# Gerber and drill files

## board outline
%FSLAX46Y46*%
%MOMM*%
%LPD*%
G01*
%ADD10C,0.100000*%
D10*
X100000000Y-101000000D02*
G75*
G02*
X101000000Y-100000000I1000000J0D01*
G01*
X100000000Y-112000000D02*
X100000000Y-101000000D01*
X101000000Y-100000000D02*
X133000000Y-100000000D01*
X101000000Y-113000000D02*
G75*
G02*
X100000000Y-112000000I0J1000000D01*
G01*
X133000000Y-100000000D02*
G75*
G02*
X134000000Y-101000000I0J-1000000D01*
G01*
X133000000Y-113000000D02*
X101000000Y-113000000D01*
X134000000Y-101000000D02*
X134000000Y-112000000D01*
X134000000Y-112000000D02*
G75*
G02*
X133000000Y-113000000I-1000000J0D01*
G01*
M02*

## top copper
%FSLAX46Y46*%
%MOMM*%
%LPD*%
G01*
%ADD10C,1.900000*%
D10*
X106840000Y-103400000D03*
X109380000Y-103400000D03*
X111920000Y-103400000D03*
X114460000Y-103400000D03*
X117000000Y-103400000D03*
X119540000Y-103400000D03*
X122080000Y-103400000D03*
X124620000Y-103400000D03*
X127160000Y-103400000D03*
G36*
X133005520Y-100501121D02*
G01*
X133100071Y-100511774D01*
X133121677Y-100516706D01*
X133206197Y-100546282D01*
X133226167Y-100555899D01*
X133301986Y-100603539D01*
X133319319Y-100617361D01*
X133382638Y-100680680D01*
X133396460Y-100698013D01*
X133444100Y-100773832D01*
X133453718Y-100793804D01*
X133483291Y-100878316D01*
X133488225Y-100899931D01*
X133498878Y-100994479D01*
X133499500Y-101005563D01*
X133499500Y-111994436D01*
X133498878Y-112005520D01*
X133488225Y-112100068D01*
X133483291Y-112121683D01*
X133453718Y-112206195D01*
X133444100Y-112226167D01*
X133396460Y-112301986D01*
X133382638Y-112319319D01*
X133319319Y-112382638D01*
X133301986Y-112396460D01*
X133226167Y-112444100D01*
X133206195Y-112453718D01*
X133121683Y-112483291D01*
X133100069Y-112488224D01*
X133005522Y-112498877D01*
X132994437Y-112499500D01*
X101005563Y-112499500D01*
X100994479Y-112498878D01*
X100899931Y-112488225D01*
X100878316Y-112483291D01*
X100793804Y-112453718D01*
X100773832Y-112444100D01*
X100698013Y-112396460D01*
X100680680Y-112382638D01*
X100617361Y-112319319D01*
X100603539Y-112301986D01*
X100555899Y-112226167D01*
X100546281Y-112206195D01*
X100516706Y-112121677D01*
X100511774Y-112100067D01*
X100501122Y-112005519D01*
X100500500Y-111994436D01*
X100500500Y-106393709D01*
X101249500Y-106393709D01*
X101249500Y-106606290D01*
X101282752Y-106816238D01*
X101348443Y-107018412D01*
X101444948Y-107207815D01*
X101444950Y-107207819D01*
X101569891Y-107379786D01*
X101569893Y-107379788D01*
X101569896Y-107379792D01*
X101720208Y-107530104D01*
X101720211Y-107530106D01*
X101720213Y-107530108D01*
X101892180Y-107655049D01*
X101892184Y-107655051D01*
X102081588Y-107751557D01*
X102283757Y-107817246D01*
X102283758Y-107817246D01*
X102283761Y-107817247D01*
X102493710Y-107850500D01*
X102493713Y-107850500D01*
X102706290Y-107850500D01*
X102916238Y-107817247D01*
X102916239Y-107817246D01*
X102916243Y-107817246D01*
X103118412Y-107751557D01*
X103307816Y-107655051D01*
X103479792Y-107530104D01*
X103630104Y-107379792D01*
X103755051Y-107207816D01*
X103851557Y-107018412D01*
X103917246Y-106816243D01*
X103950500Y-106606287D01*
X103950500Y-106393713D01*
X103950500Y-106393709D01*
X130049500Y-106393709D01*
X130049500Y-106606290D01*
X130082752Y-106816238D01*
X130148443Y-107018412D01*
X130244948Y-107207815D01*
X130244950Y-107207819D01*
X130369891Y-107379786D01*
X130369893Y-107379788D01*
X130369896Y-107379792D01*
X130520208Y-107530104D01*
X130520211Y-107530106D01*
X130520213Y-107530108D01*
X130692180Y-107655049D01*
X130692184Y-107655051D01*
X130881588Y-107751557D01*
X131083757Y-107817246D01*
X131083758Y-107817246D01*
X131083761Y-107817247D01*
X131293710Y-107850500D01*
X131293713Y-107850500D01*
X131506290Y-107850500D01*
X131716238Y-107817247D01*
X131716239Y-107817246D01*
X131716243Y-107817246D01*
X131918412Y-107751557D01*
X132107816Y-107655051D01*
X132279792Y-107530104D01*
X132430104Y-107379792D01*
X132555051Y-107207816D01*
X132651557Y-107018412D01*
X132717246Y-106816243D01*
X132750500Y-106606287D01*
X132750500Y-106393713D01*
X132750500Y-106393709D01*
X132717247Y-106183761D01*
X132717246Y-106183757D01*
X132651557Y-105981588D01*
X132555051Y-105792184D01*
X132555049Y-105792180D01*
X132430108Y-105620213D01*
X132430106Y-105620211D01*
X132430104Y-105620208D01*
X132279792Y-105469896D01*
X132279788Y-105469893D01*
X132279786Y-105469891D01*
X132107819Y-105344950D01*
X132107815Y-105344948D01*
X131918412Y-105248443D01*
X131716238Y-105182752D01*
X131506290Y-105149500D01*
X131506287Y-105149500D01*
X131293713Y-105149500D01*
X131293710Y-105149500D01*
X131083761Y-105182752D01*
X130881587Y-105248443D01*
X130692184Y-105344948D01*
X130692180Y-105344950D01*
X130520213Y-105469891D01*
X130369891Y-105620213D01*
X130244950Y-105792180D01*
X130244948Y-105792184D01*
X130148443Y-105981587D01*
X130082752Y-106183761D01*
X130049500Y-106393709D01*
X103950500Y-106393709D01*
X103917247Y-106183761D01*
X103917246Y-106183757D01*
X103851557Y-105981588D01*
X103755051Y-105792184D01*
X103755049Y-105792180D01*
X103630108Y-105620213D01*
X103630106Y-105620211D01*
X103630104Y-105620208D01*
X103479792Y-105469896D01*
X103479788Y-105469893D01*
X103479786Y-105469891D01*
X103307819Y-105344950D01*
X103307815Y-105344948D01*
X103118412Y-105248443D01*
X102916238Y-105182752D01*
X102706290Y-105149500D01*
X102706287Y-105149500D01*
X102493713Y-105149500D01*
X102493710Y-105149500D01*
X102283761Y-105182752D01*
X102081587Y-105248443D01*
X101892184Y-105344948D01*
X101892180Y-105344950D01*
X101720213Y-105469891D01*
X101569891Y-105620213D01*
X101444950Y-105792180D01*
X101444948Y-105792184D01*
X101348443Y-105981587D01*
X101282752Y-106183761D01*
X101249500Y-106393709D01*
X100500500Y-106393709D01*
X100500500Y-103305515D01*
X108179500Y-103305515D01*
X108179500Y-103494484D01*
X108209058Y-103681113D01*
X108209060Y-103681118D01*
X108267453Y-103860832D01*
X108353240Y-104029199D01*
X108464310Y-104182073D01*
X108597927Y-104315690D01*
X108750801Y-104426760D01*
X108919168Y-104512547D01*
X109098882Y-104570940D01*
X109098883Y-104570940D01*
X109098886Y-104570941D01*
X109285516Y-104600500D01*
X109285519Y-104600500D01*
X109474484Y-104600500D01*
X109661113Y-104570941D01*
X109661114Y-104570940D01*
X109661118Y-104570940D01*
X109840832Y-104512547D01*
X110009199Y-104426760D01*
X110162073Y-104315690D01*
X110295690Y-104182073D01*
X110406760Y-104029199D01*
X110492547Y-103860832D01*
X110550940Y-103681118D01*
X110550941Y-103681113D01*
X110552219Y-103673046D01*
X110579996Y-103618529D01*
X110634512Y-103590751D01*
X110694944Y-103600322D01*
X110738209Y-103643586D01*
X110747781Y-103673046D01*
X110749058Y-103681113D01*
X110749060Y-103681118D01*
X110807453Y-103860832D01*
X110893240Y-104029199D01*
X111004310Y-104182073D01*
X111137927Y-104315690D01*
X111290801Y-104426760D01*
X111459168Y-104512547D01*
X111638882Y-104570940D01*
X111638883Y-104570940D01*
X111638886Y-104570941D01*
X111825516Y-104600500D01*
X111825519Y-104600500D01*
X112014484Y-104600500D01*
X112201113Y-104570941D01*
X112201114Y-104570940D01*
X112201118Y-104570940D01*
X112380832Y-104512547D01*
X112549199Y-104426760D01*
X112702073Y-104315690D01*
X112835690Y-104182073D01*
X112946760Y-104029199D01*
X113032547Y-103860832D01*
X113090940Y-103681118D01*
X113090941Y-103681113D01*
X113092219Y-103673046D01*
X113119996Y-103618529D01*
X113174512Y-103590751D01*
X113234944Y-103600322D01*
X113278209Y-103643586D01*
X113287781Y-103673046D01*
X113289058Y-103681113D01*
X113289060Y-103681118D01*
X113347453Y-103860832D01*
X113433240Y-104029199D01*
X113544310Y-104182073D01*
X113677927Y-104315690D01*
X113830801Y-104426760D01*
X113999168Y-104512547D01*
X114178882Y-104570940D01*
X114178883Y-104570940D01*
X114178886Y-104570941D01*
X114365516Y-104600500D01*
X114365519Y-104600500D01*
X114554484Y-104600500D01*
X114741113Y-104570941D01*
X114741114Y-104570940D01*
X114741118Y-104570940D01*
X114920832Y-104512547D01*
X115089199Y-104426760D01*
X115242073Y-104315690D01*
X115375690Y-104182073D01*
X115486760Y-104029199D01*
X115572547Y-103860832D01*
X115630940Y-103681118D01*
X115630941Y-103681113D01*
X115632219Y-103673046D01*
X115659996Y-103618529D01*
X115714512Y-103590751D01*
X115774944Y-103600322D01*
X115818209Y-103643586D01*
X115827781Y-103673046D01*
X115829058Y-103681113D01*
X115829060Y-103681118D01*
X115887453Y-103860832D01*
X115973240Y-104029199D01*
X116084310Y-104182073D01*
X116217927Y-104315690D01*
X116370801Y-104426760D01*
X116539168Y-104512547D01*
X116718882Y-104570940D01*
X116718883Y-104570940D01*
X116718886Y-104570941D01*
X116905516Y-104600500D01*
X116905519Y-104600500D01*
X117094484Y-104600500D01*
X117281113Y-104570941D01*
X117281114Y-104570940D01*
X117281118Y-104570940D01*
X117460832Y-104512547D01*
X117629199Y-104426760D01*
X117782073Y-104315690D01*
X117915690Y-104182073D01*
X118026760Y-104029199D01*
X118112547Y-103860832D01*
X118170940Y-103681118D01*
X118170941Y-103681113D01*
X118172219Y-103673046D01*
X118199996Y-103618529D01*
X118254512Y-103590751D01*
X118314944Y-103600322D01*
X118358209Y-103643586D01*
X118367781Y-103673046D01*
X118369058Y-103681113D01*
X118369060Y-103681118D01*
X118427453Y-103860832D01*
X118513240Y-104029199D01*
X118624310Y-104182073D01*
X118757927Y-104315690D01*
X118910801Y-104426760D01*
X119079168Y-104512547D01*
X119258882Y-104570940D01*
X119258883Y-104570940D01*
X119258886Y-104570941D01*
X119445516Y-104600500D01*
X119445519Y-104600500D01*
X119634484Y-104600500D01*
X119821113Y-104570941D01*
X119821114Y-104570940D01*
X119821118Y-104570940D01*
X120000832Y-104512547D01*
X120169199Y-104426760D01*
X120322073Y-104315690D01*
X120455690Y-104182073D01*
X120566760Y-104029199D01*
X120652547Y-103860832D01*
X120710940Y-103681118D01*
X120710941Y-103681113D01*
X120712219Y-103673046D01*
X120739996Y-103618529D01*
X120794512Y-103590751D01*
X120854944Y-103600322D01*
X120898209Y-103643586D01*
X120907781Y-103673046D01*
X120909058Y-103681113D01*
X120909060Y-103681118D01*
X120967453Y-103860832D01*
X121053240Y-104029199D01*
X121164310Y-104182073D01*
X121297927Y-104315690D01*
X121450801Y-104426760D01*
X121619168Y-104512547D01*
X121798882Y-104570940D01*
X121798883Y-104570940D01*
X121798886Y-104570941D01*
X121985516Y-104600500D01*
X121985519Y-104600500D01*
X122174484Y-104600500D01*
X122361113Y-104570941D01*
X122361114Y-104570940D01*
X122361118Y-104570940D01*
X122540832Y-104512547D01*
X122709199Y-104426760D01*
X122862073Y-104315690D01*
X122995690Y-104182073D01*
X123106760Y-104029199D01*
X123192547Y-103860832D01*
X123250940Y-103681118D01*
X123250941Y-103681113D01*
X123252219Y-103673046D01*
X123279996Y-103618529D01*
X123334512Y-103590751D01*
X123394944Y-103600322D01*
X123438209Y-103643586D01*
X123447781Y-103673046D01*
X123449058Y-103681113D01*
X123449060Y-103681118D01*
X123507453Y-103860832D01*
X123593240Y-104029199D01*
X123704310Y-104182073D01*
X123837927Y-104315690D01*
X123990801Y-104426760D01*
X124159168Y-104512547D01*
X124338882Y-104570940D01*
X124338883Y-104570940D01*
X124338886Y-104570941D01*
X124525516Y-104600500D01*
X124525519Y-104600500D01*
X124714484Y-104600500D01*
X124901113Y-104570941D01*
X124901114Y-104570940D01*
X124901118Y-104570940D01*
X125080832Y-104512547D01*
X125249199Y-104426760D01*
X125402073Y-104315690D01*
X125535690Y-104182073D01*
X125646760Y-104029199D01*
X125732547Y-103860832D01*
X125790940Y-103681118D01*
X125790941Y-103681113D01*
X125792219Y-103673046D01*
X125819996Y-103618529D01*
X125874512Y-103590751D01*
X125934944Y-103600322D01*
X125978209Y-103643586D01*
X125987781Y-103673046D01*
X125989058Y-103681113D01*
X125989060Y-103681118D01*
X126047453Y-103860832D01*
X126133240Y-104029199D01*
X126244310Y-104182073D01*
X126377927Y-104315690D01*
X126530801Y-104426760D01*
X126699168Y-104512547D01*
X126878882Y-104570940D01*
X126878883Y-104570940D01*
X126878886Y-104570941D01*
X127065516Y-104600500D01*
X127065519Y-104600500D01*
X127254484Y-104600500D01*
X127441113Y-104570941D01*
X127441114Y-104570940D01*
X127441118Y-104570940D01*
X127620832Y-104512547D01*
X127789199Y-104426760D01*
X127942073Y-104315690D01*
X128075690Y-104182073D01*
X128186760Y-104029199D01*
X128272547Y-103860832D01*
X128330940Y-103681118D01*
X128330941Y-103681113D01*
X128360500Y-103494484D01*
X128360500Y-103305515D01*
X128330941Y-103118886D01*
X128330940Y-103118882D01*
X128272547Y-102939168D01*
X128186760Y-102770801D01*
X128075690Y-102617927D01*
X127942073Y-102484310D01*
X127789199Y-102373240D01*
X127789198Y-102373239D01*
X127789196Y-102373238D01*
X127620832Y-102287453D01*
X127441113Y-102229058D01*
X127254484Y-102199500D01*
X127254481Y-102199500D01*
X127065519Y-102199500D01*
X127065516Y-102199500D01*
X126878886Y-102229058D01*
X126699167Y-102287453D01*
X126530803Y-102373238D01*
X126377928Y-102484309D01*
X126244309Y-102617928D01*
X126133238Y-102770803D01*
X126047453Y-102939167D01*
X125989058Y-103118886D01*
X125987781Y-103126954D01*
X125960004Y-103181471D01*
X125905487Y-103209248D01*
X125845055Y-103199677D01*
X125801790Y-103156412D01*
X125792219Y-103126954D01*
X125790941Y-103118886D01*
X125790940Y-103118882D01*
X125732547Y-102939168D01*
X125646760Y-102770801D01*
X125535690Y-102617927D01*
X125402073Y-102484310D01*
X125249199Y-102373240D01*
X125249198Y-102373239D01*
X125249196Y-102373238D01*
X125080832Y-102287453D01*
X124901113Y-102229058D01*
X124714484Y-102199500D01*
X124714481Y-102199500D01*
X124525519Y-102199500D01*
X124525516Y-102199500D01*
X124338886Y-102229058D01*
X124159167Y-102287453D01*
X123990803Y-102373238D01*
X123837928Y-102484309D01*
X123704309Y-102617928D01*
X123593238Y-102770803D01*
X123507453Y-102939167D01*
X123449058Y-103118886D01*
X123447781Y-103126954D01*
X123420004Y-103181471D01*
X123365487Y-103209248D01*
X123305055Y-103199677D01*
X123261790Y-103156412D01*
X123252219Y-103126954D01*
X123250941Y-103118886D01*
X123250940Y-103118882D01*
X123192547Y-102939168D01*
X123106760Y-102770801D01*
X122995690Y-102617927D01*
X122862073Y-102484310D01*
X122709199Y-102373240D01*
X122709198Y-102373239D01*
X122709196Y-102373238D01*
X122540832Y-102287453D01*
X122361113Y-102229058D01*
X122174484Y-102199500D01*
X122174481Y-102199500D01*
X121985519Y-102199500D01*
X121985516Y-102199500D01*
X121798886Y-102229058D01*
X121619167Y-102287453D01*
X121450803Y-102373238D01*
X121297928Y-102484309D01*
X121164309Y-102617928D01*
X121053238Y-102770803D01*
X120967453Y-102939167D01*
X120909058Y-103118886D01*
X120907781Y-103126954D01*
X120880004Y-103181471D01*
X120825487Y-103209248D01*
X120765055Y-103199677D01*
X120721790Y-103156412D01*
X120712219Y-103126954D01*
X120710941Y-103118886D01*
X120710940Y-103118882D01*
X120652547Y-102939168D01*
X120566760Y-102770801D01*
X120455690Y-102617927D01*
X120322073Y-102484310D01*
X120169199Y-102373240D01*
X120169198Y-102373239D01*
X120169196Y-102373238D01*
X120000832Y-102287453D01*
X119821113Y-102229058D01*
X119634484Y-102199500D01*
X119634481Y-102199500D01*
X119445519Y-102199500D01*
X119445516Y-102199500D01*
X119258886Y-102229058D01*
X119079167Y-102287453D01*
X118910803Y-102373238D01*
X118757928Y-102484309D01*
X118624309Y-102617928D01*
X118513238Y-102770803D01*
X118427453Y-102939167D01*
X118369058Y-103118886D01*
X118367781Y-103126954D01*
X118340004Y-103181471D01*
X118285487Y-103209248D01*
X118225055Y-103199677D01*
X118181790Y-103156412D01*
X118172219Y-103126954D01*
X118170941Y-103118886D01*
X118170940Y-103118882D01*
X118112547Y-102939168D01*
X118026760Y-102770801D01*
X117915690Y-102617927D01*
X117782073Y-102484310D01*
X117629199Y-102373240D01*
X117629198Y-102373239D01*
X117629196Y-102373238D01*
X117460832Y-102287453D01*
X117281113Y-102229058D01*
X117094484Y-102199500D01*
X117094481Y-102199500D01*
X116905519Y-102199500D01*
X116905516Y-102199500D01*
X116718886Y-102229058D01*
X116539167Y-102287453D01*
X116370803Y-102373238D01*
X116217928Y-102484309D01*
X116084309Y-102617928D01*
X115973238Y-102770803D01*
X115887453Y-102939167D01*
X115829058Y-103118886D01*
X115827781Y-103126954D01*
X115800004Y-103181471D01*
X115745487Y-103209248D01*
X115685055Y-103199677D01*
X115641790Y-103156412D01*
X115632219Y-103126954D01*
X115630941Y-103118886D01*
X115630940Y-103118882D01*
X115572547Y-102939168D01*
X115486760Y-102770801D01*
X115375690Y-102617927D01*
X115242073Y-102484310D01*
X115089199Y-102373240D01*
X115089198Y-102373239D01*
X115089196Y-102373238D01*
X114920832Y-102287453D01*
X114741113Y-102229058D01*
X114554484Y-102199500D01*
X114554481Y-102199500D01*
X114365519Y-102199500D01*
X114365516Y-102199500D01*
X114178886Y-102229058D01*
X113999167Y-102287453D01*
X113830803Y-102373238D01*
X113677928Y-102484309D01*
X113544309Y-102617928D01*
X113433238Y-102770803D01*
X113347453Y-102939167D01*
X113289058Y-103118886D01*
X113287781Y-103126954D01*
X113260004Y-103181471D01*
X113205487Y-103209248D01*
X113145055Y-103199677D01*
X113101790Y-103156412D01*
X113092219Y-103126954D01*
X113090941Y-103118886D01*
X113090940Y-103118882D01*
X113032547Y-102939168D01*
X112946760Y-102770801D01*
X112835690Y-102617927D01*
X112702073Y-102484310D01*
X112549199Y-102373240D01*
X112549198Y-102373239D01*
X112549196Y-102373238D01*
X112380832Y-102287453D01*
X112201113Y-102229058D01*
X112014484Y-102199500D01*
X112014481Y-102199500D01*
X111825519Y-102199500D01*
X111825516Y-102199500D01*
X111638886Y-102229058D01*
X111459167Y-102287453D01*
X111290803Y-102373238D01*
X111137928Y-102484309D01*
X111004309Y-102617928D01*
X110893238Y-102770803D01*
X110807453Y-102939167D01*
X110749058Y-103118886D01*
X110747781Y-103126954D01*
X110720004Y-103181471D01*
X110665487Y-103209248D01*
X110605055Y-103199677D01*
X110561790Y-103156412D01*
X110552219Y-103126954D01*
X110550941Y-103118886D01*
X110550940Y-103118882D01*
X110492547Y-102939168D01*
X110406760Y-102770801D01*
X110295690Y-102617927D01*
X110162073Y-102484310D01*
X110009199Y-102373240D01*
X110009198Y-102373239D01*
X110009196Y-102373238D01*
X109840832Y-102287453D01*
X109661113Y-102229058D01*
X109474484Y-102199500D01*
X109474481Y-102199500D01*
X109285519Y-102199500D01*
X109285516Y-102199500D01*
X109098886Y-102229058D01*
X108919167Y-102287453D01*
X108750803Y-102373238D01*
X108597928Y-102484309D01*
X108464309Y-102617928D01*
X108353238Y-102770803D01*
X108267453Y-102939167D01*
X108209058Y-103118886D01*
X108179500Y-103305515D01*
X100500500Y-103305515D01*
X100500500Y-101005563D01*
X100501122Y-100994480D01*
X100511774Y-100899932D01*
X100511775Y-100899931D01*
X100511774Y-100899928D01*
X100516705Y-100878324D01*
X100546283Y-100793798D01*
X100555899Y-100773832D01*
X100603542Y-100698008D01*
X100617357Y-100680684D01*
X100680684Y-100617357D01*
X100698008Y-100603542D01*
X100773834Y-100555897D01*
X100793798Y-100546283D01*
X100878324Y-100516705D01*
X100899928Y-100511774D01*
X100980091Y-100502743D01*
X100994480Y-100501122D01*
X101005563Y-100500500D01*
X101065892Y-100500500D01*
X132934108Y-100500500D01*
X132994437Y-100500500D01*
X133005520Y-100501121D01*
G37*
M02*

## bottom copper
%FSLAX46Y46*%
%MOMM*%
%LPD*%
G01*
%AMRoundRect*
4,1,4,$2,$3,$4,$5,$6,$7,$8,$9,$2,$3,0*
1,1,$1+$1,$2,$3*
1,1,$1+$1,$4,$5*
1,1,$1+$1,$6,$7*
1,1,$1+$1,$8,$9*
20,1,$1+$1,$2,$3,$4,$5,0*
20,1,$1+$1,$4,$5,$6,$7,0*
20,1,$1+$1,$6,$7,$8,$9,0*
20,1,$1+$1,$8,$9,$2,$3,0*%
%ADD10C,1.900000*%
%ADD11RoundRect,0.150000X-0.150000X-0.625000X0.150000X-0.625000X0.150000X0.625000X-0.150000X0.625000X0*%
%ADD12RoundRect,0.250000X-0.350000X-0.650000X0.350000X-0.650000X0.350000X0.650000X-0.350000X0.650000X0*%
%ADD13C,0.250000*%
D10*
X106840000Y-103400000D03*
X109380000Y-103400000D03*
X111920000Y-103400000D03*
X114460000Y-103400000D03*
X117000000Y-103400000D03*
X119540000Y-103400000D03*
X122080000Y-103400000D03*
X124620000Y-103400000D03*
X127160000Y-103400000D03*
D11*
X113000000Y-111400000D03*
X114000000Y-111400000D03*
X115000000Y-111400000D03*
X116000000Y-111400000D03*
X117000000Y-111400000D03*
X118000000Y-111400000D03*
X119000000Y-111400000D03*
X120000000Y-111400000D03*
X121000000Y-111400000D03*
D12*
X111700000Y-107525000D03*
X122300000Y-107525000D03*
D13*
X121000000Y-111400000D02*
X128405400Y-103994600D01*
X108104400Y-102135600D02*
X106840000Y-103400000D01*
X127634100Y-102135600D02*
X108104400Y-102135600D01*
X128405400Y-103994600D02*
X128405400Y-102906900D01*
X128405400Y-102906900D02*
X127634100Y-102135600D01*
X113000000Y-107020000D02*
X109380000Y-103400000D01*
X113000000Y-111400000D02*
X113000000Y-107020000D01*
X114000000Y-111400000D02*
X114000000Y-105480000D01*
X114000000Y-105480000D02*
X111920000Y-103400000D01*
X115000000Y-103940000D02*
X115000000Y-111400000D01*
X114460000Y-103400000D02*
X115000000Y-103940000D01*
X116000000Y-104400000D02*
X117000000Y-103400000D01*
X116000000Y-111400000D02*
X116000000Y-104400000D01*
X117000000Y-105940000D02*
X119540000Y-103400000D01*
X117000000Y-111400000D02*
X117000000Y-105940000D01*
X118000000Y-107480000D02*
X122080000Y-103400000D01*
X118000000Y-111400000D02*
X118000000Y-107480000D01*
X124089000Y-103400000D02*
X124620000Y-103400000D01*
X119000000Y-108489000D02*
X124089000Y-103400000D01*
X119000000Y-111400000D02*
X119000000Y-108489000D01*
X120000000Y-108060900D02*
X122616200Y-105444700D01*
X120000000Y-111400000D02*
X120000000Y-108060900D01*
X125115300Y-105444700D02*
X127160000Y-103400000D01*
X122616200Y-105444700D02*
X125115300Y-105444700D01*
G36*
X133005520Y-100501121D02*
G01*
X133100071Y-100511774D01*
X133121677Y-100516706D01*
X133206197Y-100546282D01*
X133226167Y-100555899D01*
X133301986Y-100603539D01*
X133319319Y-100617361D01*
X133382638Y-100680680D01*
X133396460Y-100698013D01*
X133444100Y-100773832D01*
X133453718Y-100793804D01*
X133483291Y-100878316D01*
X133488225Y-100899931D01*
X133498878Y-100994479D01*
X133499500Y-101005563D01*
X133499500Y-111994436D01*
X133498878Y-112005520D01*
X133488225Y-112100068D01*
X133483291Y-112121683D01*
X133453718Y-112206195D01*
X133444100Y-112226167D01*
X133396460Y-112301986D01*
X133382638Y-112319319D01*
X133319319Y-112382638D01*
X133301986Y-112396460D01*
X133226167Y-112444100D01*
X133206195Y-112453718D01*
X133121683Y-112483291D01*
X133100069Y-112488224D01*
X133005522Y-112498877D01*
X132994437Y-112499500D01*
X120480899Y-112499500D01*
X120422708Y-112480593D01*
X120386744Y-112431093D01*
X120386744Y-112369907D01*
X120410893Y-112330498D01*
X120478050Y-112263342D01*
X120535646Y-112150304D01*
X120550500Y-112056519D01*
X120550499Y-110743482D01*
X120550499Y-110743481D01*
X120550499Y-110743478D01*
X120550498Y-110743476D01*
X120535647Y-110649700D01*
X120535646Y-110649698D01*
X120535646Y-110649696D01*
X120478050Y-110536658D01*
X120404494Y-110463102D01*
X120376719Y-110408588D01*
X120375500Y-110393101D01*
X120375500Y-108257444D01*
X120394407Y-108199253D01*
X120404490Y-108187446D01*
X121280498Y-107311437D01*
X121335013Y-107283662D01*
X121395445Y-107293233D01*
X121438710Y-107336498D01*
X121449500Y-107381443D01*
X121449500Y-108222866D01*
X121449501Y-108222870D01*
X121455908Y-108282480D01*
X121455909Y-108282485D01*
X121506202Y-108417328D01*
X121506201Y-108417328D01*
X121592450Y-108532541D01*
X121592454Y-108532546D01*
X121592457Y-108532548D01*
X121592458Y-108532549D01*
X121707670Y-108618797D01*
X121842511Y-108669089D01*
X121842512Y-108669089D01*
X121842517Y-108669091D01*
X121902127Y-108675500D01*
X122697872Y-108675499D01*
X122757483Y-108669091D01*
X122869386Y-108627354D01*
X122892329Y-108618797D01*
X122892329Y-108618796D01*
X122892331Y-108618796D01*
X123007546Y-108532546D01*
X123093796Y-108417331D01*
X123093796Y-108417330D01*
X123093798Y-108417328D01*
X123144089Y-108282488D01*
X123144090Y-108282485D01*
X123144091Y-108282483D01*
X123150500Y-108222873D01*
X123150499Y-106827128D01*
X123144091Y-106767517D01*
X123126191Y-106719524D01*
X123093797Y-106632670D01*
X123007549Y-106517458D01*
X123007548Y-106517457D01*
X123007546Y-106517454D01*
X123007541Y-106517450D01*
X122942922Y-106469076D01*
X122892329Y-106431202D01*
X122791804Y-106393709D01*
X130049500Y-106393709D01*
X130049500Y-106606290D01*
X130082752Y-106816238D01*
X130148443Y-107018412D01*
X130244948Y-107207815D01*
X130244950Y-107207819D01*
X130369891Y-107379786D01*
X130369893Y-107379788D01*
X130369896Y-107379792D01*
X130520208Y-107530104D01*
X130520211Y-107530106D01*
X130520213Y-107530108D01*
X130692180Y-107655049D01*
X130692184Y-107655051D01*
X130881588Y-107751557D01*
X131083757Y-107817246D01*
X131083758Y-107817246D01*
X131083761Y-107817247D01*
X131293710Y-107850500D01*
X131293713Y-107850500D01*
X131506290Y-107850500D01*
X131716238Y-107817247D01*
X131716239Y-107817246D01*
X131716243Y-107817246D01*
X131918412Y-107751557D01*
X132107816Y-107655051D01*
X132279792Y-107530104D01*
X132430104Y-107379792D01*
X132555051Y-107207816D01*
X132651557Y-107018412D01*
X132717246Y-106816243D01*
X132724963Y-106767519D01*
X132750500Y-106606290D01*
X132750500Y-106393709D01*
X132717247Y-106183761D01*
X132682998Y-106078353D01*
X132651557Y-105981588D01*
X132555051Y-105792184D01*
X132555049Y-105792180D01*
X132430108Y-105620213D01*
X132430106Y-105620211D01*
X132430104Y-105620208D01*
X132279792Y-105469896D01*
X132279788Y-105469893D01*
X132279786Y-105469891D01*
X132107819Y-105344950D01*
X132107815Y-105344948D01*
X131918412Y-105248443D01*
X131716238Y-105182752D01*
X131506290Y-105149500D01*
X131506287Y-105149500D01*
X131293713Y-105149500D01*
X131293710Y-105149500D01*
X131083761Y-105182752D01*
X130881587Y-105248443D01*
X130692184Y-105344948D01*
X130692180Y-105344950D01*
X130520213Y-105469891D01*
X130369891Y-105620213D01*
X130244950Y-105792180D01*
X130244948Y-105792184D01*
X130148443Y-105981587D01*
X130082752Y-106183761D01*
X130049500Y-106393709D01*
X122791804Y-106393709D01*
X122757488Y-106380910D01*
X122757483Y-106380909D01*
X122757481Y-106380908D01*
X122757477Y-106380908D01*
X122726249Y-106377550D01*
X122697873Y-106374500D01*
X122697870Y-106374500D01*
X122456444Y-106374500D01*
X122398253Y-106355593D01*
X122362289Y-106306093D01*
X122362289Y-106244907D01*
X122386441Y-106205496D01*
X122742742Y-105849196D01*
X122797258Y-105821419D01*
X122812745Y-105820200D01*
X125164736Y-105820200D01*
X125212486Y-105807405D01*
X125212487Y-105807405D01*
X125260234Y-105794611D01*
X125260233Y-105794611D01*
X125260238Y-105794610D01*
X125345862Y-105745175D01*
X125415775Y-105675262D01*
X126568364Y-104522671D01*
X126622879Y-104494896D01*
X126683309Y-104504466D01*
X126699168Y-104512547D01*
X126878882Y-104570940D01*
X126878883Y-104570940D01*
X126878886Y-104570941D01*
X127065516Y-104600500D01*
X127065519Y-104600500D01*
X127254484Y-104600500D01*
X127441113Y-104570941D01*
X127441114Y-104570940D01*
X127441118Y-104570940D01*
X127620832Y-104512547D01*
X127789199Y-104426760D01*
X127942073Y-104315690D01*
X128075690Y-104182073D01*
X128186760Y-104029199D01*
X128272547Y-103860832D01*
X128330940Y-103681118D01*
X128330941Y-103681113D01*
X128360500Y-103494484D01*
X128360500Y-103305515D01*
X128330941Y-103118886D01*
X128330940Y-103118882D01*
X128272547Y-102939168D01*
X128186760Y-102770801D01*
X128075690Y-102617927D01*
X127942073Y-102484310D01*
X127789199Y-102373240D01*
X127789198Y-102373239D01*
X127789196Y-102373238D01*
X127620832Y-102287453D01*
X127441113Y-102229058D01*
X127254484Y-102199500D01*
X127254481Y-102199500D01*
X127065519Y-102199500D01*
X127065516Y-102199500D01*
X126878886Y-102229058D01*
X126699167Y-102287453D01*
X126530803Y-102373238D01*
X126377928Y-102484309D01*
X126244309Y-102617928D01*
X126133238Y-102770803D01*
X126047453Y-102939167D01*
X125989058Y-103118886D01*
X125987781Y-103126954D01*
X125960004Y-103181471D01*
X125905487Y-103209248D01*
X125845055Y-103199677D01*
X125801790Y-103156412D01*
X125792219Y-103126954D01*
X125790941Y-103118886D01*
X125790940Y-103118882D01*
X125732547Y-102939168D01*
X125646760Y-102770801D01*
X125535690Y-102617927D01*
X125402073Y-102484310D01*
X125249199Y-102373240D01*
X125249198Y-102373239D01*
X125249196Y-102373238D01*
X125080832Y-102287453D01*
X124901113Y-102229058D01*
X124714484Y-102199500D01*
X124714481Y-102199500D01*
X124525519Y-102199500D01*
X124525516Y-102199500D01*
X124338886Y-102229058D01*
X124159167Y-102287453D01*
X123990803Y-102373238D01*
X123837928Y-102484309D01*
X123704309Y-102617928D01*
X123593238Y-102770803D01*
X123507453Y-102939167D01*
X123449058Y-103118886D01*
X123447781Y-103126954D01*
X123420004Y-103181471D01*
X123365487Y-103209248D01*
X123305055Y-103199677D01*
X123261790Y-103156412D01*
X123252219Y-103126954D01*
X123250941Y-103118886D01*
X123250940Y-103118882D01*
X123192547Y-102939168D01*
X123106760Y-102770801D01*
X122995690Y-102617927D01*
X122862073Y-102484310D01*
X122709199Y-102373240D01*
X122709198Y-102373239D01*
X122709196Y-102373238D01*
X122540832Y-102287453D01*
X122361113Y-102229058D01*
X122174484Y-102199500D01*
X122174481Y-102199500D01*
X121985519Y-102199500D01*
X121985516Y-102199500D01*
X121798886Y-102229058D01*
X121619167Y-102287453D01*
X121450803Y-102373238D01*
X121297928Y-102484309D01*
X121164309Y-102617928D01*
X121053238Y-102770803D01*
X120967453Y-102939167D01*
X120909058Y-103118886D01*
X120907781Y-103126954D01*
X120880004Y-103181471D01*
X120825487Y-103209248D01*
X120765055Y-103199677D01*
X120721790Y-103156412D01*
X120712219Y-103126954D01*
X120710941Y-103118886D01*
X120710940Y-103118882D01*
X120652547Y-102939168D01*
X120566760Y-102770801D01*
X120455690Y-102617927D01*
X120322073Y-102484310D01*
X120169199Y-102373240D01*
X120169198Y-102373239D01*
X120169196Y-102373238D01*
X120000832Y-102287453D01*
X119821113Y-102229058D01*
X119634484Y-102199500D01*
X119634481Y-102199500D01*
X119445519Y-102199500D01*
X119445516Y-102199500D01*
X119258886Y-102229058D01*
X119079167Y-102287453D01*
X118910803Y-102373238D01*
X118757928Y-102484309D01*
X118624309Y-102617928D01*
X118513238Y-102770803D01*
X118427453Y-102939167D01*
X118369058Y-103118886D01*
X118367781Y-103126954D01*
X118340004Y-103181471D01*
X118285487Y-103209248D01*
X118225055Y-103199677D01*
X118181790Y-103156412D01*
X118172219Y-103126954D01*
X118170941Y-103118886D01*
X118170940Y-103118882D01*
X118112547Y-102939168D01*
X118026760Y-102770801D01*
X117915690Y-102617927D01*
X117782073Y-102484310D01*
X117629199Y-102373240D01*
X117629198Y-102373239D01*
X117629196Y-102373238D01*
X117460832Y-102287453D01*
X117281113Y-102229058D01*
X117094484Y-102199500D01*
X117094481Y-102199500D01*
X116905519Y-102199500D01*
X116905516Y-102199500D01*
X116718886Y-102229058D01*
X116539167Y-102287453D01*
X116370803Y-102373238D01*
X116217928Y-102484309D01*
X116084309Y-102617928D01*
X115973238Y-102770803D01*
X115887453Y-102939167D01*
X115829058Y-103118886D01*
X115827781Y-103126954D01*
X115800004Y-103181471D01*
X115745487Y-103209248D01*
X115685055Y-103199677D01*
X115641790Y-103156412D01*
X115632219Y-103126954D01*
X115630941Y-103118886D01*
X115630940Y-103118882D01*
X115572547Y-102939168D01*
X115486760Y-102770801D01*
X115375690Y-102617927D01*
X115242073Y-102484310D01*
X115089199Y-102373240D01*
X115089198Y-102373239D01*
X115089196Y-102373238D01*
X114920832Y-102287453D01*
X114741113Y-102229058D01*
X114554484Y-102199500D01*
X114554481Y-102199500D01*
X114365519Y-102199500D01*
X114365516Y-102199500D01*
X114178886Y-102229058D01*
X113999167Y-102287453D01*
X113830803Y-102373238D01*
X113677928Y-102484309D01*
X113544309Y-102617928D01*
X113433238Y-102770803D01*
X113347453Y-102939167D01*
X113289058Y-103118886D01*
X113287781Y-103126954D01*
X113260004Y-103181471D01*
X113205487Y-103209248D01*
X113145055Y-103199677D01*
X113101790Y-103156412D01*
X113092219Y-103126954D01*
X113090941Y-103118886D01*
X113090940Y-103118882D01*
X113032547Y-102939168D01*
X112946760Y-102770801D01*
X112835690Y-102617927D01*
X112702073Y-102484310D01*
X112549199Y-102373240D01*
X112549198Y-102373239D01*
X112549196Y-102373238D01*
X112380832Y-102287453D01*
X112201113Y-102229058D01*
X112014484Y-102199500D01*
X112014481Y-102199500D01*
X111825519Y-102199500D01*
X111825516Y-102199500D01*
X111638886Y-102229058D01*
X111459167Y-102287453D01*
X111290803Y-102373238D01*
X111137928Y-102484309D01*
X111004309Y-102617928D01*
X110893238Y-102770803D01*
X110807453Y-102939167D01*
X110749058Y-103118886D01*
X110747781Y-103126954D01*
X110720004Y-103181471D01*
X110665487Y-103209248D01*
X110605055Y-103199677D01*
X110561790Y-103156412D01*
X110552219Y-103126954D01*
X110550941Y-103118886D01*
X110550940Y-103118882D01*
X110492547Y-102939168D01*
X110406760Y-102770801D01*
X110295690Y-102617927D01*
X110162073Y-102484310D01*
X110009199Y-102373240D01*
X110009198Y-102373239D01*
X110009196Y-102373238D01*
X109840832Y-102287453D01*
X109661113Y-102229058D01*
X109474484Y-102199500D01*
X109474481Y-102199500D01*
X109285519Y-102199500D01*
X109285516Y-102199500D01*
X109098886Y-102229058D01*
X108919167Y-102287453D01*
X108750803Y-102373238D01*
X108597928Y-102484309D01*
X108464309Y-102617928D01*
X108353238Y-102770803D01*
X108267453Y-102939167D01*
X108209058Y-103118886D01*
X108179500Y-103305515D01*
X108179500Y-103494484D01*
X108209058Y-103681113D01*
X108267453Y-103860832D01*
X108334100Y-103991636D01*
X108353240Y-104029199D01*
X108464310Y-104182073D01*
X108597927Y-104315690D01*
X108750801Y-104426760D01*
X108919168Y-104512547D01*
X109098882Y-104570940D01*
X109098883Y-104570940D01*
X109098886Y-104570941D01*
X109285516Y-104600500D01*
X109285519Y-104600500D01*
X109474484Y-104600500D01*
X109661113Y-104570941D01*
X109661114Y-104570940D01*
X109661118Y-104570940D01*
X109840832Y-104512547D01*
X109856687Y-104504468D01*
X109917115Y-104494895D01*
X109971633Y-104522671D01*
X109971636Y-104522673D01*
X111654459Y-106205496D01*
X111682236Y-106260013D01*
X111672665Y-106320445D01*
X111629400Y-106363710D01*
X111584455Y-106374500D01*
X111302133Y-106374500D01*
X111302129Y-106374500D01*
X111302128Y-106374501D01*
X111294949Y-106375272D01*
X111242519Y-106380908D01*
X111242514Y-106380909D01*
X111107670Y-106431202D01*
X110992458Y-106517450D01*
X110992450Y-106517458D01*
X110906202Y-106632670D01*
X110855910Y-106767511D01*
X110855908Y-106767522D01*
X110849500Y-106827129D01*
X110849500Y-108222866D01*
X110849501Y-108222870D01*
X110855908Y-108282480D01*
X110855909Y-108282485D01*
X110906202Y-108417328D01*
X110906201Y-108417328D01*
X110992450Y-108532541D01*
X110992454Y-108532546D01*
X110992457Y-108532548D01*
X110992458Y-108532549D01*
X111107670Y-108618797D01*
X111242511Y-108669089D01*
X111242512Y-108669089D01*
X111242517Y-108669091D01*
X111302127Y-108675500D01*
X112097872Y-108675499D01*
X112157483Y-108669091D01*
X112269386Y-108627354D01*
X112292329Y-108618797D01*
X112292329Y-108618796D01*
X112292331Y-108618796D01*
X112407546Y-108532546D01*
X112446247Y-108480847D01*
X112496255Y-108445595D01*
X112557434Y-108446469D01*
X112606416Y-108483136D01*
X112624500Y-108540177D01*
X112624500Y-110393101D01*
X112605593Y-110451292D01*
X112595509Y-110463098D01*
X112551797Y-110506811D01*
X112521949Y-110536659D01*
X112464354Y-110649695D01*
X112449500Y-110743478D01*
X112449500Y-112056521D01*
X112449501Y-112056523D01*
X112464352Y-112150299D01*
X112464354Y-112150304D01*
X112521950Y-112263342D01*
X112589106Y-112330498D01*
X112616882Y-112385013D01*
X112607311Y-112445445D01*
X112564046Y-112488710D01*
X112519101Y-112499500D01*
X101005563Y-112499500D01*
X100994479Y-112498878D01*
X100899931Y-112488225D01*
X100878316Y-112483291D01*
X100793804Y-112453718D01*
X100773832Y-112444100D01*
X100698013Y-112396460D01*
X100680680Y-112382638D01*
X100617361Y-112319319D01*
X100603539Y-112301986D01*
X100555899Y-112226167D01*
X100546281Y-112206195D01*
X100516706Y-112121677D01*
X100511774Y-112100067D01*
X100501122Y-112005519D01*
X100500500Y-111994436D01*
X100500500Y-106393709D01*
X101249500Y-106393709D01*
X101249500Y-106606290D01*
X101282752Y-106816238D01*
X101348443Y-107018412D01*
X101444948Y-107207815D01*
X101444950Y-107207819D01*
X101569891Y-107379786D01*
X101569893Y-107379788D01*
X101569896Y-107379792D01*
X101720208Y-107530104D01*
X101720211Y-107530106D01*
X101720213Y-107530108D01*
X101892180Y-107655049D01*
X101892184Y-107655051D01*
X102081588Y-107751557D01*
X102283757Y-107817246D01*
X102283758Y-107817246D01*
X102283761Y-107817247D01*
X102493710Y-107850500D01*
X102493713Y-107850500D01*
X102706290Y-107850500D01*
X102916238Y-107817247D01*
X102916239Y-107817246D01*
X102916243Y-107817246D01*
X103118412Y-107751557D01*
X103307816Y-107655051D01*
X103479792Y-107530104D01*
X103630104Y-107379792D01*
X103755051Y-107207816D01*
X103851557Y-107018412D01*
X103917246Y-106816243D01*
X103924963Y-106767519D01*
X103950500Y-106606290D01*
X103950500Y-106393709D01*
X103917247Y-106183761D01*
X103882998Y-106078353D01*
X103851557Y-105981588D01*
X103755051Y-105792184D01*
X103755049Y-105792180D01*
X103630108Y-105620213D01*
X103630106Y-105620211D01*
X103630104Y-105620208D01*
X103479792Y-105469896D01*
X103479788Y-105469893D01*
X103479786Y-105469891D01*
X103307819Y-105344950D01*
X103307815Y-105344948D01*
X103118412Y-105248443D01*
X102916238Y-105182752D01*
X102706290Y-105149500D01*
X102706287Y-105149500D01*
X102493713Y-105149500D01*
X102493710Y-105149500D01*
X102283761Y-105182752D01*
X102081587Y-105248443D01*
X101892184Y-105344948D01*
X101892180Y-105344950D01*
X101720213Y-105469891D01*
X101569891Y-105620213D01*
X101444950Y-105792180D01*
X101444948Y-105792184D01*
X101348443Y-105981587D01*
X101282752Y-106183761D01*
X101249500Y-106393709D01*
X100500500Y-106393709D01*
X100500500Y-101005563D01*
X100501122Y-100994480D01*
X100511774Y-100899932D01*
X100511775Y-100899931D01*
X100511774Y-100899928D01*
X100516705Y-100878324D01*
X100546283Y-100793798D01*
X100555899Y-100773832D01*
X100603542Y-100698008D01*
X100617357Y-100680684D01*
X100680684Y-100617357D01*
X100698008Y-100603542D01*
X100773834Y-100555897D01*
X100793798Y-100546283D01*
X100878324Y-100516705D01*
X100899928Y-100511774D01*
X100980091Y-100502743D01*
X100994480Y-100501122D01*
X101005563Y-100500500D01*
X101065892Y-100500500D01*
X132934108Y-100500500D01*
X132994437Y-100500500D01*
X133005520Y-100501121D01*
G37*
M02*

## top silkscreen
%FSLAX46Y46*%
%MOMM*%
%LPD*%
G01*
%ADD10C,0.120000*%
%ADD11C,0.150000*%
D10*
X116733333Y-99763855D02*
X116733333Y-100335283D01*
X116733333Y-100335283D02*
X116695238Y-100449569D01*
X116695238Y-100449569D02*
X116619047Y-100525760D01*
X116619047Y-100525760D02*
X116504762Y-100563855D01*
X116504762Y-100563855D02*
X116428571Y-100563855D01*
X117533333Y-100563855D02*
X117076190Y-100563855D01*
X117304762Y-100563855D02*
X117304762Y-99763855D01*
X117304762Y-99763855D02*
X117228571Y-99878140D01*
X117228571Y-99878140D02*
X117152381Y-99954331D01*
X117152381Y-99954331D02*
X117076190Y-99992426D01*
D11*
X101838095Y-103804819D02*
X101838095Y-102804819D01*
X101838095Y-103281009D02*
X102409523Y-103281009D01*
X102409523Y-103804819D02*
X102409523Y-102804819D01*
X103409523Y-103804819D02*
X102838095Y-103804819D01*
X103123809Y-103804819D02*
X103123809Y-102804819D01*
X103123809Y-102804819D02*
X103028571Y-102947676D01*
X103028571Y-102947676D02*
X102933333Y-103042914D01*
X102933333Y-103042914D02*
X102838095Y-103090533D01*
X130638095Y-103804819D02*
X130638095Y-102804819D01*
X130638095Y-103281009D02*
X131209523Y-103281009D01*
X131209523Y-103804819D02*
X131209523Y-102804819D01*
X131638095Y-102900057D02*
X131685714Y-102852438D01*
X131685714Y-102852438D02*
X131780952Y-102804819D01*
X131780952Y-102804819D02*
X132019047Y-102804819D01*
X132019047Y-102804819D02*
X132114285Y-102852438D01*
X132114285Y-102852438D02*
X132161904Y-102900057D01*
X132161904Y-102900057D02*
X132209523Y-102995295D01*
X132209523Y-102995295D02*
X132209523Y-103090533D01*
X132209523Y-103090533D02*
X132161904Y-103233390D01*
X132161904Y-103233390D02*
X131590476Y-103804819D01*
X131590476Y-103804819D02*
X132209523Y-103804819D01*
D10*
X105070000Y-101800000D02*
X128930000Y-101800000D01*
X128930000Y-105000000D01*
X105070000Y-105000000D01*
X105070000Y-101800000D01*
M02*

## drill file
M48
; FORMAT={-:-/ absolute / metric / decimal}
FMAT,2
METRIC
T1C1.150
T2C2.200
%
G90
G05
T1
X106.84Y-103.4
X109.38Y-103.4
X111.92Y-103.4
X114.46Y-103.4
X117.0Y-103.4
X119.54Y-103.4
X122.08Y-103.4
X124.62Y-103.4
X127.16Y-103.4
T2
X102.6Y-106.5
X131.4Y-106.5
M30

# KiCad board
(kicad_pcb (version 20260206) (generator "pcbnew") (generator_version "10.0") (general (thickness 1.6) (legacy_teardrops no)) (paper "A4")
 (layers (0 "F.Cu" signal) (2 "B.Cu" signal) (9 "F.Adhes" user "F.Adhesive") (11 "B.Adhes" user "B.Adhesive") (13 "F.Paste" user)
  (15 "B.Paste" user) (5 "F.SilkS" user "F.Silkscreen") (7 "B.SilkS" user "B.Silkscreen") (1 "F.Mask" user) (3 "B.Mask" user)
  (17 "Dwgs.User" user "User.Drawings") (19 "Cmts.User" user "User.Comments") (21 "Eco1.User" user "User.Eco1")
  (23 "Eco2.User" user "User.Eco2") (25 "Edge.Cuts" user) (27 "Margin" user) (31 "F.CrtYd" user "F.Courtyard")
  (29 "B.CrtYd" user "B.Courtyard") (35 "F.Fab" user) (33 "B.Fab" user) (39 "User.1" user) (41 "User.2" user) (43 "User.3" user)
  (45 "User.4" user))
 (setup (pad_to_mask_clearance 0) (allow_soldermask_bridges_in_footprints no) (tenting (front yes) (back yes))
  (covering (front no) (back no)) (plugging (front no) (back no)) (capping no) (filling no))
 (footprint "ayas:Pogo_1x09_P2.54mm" (layer "F.Cu") (at 117 103.4)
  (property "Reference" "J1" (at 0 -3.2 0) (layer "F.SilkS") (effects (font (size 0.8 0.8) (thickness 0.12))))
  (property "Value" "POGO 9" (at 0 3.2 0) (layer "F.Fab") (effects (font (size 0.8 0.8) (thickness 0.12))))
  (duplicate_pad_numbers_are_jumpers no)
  (fp_rect (start -11.93 -1.6) (end 11.93 1.6) (stroke (width 0.12) (type solid)) (fill no) (layer "F.SilkS"))
  (pad "1" thru_hole circle (at -10.16 0) (size 1.9 1.9) (drill 1.15) (layers "*.Cu" "*.Mask") (remove_unused_layers no) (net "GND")
   (zone_connect 2))
  (pad "2" thru_hole circle (at -7.62 0) (size 1.9 1.9) (drill 1.15) (layers "*.Cu" "*.Mask") (remove_unused_layers no) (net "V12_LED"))
  (pad "3" thru_hole circle (at -5.08 0) (size 1.9 1.9) (drill 1.15) (layers "*.Cu" "*.Mask") (remove_unused_layers no) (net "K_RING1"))
  (pad "4" thru_hole circle (at -2.54 0) (size 1.9 1.9) (drill 1.15) (layers "*.Cu" "*.Mask") (remove_unused_layers no) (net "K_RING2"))
  (pad "5" thru_hole circle (at 0 0) (size 1.9 1.9) (drill 1.15) (layers "*.Cu" "*.Mask") (remove_unused_layers no) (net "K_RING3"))
  (pad "6" thru_hole circle (at 2.54 0) (size 1.9 1.9) (drill 1.15) (layers "*.Cu" "*.Mask") (remove_unused_layers no) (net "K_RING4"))
  (pad "7" thru_hole circle (at 5.08 0) (size 1.9 1.9) (drill 1.15) (layers "*.Cu" "*.Mask") (remove_unused_layers no) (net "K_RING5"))
  (pad "8" thru_hole circle (at 7.62 0) (size 1.9 1.9) (drill 1.15) (layers "*.Cu" "*.Mask") (remove_unused_layers no) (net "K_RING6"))
  (pad "9" thru_hole circle (at 10.16 0) (size 1.9 1.9) (drill 1.15) (layers "*.Cu" "*.Mask") (remove_unused_layers no) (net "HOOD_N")))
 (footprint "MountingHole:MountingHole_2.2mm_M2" (layer "F.Cu") (at 102.6 106.5)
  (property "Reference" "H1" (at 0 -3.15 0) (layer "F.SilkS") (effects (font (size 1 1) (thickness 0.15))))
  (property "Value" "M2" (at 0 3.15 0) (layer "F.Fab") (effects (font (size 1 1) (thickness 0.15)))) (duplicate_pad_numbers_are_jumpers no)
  (pad "" np_thru_hole circle (at 0 0) (size 2.2 2.2) (drill 2.2) (layers "*.Cu" "*.Mask") (zone_connect 2)))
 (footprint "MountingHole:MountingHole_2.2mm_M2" (layer "F.Cu") (at 131.4 106.5)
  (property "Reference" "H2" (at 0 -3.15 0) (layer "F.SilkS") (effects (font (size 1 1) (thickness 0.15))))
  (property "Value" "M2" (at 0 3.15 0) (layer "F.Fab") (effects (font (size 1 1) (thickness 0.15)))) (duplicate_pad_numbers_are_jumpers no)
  (pad "" np_thru_hole circle (at 0 0) (size 2.2 2.2) (drill 2.2) (layers "*.Cu" "*.Mask") (zone_connect 2)))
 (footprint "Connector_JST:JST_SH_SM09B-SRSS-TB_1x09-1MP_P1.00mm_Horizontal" (layer "B.Cu") (at 117 109.4)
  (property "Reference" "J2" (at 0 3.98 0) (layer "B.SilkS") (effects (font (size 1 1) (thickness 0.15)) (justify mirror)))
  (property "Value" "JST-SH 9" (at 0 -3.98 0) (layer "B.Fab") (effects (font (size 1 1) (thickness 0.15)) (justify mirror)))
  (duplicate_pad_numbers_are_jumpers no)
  (pad "1" smd roundrect (at -4 2) (size 0.6 1.55) (layers "B.Cu" "B.Mask" "B.Paste") (roundrect_rratio 0.25) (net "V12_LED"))
  (pad "2" smd roundrect (at -3 2) (size 0.6 1.55) (layers "B.Cu" "B.Mask" "B.Paste") (roundrect_rratio 0.25) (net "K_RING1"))
  (pad "3" smd roundrect (at -2 2) (size 0.6 1.55) (layers "B.Cu" "B.Mask" "B.Paste") (roundrect_rratio 0.25) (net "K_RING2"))
  (pad "4" smd roundrect (at -1 2) (size 0.6 1.55) (layers "B.Cu" "B.Mask" "B.Paste") (roundrect_rratio 0.25) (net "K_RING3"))
  (pad "5" smd roundrect (at 0 2) (size 0.6 1.55) (layers "B.Cu" "B.Mask" "B.Paste") (roundrect_rratio 0.25) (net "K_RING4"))
  (pad "6" smd roundrect (at 1 2) (size 0.6 1.55) (layers "B.Cu" "B.Mask" "B.Paste") (roundrect_rratio 0.25) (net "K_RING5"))
  (pad "7" smd roundrect (at 2 2) (size 0.6 1.55) (layers "B.Cu" "B.Mask" "B.Paste") (roundrect_rratio 0.25) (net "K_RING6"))
  (pad "8" smd roundrect (at 3 2) (size 0.6 1.55) (layers "B.Cu" "B.Mask" "B.Paste") (roundrect_rratio 0.25) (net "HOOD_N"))
  (pad "9" smd roundrect (at 4 2) (size 0.6 1.55) (layers "B.Cu" "B.Mask" "B.Paste") (roundrect_rratio 0.25) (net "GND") (zone_connect 2))
  (pad "MP" smd roundrect (at -5.3 -1.875) (size 1.2 1.8) (layers "B.Cu" "B.Mask" "B.Paste") (roundrect_rratio 0.208333) (zone_connect 2))
  (pad "MP" smd roundrect (at 5.3 -1.875) (size 1.2 1.8) (layers "B.Cu" "B.Mask" "B.Paste") (roundrect_rratio 0.208333) (zone_connect 2)))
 (gr_arc (start 100 101) (mid 100.292893 100.292893) (end 101 100) (stroke (width 0.1) (type default)) (layer "Edge.Cuts"))
 (gr_line (start 100 112) (end 100 101) (stroke (width 0.1) (type default)) (layer "Edge.Cuts"))
 (gr_line (start 101 100) (end 133 100) (stroke (width 0.1) (type default)) (layer "Edge.Cuts"))
 (gr_arc (start 101 113) (mid 100.292893 112.707107) (end 100 112) (stroke (width 0.1) (type default)) (layer "Edge.Cuts"))
 (gr_arc (start 133 100) (mid 133.707107 100.292893) (end 134 101) (stroke (width 0.1) (type default)) (layer "Edge.Cuts"))
 (gr_line (start 133 113) (end 101 113) (stroke (width 0.1) (type default)) (layer "Edge.Cuts"))
 (gr_line (start 134 101) (end 134 112) (stroke (width 0.1) (type default)) (layer "Edge.Cuts"))
 (gr_arc (start 134 112) (mid 133.707107 112.707107) (end 133 113) (stroke (width 0.1) (type default)) (layer "Edge.Cuts"))
 (segment (start 121 111.4) (end 128.4054 103.9946) (width 0.25) (layer "B.Cu") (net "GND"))
 (segment (start 108.1044 102.1356) (end 106.84 103.4) (width 0.25) (layer "B.Cu") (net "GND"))
 (segment (start 127.6341 102.1356) (end 108.1044 102.1356) (width 0.25) (layer "B.Cu") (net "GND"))
 (segment (start 128.4054 103.9946) (end 128.4054 102.9069) (width 0.25) (layer "B.Cu") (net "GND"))
 (segment (start 128.4054 102.9069) (end 127.6341 102.1356) (width 0.25) (layer "B.Cu") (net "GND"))
 (segment (start 113 107.02) (end 109.38 103.4) (width 0.25) (layer "B.Cu") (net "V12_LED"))
 (segment (start 113 111.4) (end 113 107.02) (width 0.25) (layer "B.Cu") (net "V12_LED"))
 (segment (start 114 111.4) (end 114 105.48) (width 0.25) (layer "B.Cu") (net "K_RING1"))
 (segment (start 114 105.48) (end 111.92 103.4) (width 0.25) (layer "B.Cu") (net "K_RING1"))
 (segment (start 115 103.94) (end 115 111.4) (width 0.25) (layer "B.Cu") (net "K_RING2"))
 (segment (start 114.46 103.4) (end 115 103.94) (width 0.25) (layer "B.Cu") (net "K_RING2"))
 (segment (start 116 104.4) (end 117 103.4) (width 0.25) (layer "B.Cu") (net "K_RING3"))
 (segment (start 116 111.4) (end 116 104.4) (width 0.25) (layer "B.Cu") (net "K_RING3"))
 (segment (start 117 105.94) (end 119.54 103.4) (width 0.25) (layer "B.Cu") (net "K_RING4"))
 (segment (start 117 111.4) (end 117 105.94) (width 0.25) (layer "B.Cu") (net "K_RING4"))
 (segment (start 118 107.48) (end 122.08 103.4) (width 0.25) (layer "B.Cu") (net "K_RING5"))
 (segment (start 118 111.4) (end 118 107.48) (width 0.25) (layer "B.Cu") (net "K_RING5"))
 (segment (start 124.089 103.4) (end 124.62 103.4) (width 0.25) (layer "B.Cu") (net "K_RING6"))
 (segment (start 119 108.489) (end 124.089 103.4) (width 0.25) (layer "B.Cu") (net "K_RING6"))
 (segment (start 119 111.4) (end 119 108.489) (width 0.25) (layer "B.Cu") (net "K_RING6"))
 (segment (start 120 108.0609) (end 122.6162 105.4447) (width 0.25) (layer "B.Cu") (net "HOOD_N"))
 (segment (start 120 111.4) (end 120 108.0609) (width 0.25) (layer "B.Cu") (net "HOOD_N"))
 (segment (start 125.1153 105.4447) (end 127.16 103.4) (width 0.25) (layer "B.Cu") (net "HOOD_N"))
 (segment (start 122.6162 105.4447) (end 125.1153 105.4447) (width 0.25) (layer "B.Cu") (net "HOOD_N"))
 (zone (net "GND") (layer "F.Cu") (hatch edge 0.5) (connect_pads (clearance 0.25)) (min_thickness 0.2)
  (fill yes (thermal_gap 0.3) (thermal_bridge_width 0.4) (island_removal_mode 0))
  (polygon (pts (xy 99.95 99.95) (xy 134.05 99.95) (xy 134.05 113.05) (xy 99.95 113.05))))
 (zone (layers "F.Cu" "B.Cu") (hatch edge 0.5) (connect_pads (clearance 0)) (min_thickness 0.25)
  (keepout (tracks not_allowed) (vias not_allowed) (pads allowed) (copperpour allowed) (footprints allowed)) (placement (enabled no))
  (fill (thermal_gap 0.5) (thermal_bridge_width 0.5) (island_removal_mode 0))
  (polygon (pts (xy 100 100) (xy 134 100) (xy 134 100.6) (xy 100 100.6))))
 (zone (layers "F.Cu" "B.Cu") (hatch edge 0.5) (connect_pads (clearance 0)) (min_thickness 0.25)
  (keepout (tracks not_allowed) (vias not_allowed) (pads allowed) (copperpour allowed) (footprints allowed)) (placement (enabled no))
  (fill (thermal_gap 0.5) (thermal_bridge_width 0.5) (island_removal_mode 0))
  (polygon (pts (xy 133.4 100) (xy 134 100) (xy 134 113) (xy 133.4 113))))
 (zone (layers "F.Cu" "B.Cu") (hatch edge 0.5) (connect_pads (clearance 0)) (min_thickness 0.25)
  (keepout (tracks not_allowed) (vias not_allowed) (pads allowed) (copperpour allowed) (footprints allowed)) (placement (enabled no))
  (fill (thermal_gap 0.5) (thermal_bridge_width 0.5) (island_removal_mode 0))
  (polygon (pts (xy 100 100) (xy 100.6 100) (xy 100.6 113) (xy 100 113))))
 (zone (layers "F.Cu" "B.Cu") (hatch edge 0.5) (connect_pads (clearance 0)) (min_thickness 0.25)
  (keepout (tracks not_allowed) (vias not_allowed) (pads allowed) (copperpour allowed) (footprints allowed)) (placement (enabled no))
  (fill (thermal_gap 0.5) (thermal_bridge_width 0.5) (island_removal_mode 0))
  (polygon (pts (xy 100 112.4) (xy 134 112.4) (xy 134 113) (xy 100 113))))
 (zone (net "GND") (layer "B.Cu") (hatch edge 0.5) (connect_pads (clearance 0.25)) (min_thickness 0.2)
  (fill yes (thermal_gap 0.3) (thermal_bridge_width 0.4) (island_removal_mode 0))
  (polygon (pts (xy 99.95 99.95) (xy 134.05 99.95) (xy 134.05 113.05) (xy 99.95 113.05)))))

